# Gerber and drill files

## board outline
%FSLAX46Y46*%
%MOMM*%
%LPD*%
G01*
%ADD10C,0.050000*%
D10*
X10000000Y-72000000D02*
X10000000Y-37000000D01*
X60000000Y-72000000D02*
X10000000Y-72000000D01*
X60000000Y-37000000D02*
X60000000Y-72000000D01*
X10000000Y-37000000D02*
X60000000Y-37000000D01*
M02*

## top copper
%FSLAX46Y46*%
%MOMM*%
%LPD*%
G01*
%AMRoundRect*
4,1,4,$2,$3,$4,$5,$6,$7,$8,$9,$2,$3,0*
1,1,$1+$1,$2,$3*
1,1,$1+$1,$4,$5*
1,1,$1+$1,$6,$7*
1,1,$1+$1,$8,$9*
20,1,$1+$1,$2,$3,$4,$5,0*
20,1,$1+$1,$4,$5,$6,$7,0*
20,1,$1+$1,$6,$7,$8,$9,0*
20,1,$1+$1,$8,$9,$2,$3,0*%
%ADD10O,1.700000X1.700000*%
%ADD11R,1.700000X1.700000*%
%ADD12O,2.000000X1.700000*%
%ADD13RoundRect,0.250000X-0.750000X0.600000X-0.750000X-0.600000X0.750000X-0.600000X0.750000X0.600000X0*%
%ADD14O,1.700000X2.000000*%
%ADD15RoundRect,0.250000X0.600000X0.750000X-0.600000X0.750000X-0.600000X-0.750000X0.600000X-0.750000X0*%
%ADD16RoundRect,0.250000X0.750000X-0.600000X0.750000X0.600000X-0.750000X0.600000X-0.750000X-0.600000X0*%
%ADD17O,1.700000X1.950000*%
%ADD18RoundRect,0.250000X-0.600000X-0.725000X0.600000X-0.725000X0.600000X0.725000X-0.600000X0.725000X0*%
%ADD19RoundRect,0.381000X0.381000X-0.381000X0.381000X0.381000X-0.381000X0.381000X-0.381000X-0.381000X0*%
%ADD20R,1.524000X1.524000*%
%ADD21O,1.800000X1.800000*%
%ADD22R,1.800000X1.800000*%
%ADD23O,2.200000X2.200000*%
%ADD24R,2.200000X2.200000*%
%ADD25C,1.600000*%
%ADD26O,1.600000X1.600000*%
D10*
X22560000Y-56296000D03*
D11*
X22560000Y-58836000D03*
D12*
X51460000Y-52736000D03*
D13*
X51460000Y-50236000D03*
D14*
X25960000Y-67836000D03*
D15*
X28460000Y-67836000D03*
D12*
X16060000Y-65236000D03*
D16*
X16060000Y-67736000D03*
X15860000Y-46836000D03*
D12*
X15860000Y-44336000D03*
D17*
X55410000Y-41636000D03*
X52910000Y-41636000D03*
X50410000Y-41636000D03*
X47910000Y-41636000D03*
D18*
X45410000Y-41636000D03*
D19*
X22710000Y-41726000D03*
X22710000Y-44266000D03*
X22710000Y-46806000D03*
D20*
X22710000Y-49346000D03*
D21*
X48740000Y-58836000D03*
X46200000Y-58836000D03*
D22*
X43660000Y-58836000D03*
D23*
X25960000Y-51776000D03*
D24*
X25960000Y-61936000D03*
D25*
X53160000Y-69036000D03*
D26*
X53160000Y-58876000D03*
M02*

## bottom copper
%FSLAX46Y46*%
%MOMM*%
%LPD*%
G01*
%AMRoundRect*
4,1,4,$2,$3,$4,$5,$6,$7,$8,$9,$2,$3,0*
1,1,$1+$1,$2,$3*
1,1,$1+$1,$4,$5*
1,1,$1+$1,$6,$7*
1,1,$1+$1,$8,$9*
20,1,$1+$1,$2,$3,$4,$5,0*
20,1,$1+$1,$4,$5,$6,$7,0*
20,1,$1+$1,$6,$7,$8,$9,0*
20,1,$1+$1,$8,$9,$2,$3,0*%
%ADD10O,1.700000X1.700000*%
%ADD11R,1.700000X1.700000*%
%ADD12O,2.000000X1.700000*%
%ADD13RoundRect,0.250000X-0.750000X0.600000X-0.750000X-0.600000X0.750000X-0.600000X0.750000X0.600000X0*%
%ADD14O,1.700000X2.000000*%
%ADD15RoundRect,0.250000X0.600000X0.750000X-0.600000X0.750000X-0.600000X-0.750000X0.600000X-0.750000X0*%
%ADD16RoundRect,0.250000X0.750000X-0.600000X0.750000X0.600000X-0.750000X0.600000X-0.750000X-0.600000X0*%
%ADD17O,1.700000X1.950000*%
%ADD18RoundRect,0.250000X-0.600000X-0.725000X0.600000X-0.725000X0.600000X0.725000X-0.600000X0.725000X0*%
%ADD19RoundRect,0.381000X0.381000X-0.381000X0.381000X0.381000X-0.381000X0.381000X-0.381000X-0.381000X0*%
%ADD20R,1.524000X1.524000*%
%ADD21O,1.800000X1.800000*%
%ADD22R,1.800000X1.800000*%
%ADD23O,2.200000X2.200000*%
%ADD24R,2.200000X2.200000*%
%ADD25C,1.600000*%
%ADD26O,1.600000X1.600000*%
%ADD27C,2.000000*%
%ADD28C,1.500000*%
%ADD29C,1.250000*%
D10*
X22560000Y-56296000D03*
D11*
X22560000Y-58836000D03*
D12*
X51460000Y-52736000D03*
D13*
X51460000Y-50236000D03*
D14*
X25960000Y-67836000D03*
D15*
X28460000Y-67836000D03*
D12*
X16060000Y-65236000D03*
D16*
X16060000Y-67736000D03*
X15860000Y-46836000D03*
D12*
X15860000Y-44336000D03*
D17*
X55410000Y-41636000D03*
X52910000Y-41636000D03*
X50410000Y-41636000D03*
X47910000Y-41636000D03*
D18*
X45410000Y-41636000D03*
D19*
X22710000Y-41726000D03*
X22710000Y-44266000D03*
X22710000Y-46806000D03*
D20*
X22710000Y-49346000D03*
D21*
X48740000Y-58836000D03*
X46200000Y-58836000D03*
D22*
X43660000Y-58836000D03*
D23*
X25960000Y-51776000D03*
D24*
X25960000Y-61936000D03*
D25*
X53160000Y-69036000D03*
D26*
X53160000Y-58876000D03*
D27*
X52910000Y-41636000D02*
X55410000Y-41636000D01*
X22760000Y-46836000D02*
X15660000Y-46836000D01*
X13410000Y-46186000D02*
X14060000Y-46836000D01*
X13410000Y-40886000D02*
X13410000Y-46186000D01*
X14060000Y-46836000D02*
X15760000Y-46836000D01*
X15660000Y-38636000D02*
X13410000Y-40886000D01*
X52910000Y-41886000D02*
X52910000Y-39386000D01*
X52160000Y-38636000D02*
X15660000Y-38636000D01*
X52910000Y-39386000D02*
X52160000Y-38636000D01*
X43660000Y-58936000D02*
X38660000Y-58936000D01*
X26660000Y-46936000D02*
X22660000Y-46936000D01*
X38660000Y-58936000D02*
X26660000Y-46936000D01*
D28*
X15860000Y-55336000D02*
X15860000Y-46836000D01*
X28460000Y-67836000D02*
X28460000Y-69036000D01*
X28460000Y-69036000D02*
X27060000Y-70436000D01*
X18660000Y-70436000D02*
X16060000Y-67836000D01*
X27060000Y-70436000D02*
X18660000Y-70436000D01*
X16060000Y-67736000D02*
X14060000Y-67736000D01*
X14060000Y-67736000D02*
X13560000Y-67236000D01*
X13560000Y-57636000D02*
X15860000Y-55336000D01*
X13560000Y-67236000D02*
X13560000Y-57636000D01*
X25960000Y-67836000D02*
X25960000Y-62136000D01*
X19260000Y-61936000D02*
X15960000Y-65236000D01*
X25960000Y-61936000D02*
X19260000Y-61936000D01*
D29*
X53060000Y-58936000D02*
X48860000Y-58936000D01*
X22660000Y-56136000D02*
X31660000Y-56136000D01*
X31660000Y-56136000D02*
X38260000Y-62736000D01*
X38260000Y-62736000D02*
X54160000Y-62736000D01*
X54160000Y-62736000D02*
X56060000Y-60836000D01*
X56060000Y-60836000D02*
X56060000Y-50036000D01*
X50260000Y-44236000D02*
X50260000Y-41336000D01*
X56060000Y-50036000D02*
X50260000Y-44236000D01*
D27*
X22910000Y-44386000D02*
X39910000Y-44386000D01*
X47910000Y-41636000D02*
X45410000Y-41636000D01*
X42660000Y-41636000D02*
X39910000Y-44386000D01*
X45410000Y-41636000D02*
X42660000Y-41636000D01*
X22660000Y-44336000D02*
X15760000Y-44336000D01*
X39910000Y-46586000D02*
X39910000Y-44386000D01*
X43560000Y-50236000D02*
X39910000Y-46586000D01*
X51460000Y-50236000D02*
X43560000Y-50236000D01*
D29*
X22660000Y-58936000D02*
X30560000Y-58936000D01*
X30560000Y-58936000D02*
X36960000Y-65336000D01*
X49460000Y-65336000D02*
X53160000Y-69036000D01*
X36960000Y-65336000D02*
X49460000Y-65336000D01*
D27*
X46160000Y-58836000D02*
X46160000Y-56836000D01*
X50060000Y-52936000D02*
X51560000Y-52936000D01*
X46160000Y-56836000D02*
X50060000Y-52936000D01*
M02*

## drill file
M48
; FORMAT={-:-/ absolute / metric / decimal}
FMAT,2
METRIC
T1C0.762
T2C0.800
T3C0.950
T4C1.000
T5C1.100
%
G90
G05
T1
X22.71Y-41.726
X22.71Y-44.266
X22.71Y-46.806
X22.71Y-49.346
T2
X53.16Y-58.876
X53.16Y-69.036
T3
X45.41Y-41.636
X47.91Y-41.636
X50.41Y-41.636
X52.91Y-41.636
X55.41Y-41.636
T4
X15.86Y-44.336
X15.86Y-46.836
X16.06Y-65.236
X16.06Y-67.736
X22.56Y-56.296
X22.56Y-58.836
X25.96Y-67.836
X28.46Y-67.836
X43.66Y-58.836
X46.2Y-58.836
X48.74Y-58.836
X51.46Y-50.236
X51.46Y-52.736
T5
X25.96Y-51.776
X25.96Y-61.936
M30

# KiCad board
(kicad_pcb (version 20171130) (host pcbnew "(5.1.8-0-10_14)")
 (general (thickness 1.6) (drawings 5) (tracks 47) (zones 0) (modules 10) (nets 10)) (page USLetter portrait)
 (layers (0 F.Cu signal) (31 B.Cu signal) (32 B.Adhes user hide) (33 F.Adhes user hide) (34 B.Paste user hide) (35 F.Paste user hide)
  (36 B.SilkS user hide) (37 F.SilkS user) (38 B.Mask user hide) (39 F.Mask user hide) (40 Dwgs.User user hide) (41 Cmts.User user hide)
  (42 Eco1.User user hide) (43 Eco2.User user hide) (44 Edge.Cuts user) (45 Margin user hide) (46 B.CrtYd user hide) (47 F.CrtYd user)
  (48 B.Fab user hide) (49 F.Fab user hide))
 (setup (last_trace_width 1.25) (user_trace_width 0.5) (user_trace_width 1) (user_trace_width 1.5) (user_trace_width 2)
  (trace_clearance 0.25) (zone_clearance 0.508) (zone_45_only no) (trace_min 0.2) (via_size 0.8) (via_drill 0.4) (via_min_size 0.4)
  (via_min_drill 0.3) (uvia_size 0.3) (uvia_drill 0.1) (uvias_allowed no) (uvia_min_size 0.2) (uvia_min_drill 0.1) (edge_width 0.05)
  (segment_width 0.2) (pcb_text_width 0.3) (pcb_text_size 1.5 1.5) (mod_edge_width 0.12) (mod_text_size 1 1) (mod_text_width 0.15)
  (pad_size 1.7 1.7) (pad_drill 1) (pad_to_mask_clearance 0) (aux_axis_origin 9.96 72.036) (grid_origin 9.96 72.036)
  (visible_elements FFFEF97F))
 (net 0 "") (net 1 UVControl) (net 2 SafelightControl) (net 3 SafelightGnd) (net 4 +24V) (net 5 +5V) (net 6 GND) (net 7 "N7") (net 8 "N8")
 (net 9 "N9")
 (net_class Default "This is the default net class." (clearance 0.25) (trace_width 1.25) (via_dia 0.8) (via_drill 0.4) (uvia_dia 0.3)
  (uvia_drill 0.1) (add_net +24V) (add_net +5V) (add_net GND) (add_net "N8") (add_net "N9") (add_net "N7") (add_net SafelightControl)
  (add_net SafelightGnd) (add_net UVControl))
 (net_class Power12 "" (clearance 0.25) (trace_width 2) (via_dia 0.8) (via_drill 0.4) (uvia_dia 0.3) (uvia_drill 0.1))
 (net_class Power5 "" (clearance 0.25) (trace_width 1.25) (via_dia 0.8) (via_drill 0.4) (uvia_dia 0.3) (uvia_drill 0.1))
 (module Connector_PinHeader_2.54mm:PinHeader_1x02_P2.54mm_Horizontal (layer F.Cu) (at 22.56 58.836 180)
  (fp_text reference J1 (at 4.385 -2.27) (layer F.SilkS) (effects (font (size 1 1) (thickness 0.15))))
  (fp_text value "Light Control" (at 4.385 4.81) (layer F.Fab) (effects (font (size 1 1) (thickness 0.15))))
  (pad 2 thru_hole oval (at 0 2.54 180) (size 1.7 1.7) (drill 1) (layers *.Cu *.Mask) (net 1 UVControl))
  (pad 1 thru_hole rect (at 0 0 180) (size 1.7 1.7) (drill 1) (layers *.Cu *.Mask) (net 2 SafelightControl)))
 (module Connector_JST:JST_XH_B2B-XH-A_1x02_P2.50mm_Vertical (layer F.Cu) (at 51.46 50.236 270)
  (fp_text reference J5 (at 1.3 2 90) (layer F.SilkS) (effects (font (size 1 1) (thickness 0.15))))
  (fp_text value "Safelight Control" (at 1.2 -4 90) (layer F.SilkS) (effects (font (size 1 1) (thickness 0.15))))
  (pad 2 thru_hole oval (at 2.5 0 270) (size 1.7 2) (drill 1) (layers *.Cu *.Mask) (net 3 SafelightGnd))
  (pad 1 thru_hole roundrect (at 0 0 270) (size 1.7 2) (drill 1) (layers *.Cu *.Mask) (roundrect_rratio 0.1470588235294118) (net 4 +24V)))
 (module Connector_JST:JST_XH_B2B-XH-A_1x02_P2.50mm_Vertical (layer F.Cu) (at 28.46 67.836 180)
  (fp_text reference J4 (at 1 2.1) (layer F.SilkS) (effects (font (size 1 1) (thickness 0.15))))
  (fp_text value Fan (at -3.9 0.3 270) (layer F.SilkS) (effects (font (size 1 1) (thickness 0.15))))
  (pad 2 thru_hole oval (at 2.5 0 180) (size 1.7 2) (drill 1) (layers *.Cu *.Mask) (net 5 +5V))
  (pad 1 thru_hole roundrect (at 0 0 180) (size 1.7 2) (drill 1) (layers *.Cu *.Mask) (roundrect_rratio 0.1470588235294118) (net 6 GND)))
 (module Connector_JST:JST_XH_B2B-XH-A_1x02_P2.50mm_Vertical (layer F.Cu) (at 16.06 67.736 90)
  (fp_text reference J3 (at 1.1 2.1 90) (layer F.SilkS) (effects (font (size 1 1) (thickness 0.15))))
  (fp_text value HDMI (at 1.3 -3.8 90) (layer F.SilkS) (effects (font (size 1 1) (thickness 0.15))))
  (pad 2 thru_hole oval (at 2.5 0 90) (size 1.7 2) (drill 1) (layers *.Cu *.Mask) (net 5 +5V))
  (pad 1 thru_hole roundrect (at 0 0 90) (size 1.7 2) (drill 1) (layers *.Cu *.Mask) (roundrect_rratio 0.1470588235294118) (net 6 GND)))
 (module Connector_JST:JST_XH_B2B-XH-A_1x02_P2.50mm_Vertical (layer F.Cu) (at 15.86 46.836 90)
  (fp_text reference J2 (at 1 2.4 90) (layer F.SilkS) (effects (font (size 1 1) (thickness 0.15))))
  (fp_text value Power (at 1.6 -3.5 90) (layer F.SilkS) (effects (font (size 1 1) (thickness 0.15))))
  (pad 1 thru_hole roundrect (at 0 0 90) (size 1.7 2) (drill 1) (layers *.Cu *.Mask) (roundrect_rratio 0.1470588235294118) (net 6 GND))
  (pad 2 thru_hole oval (at 2.5 0 90) (size 1.7 2) (drill 1) (layers *.Cu *.Mask) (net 4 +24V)))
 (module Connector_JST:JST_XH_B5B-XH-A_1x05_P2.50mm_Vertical (layer F.Cu) (at 45.41 41.636)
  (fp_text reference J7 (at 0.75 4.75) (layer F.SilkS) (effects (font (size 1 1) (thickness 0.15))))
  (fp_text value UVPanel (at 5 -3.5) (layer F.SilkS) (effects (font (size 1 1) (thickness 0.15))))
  (pad 5 thru_hole oval (at 10 0) (size 1.7 1.95) (drill 0.95) (layers *.Cu *.Mask) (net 6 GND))
  (pad 4 thru_hole oval (at 7.5 0) (size 1.7 1.95) (drill 0.95) (layers *.Cu *.Mask) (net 6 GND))
  (pad 3 thru_hole oval (at 5 0) (size 1.7 1.95) (drill 0.95) (layers *.Cu *.Mask) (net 1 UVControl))
  (pad 2 thru_hole oval (at 2.5 0) (size 1.7 1.95) (drill 0.95) (layers *.Cu *.Mask) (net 4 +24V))
  (pad 1 thru_hole roundrect (at 0 0) (size 1.7 1.95) (drill 0.95) (layers *.Cu *.Mask) (roundrect_rratio 0.1470588235294118) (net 4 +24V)))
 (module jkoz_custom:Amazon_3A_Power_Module (layer F.Cu) (at 30.66 45.636 90)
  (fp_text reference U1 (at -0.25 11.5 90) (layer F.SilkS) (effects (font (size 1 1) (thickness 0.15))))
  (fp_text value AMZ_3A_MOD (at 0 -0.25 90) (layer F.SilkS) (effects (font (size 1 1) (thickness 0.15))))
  (pad 4 thru_hole roundrect (at 3.91 -7.95 90) (size 1.524 1.524) (drill 0.762) (layers *.Cu *.Mask) (roundrect_rratio 0.25) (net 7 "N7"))
  (pad 3 thru_hole roundrect (at 1.37 -7.95 90) (size 1.524 1.524) (drill 0.762) (layers *.Cu *.Mask) (roundrect_rratio 0.25) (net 4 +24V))
  (pad 2 thru_hole roundrect (at -1.17 -7.95 90) (size 1.524 1.524) (drill 0.762) (layers *.Cu *.Mask) (roundrect_rratio 0.25) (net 6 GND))
  (pad 1 thru_hole rect (at -3.71 -7.95 90) (size 1.524 1.524) (drill 0.762) (layers *.Cu *.Mask) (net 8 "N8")))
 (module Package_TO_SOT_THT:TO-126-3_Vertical (layer F.Cu) (at 43.66 58.836)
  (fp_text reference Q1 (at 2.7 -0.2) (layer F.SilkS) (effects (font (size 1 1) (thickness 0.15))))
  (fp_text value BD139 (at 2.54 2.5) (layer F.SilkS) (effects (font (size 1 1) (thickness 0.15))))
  (pad 3 thru_hole oval (at 5.08 0) (size 1.8 1.8) (drill 1) (layers *.Cu *.Mask) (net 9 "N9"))
  (pad 2 thru_hole oval (at 2.54 0) (size 1.8 1.8) (drill 1) (layers *.Cu *.Mask) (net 3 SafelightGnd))
  (pad 1 thru_hole rect (at 0 0) (size 1.8 1.8) (drill 1) (layers *.Cu *.Mask) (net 6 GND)))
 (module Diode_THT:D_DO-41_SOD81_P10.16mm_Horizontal (layer F.Cu) (at 25.96 61.936 90)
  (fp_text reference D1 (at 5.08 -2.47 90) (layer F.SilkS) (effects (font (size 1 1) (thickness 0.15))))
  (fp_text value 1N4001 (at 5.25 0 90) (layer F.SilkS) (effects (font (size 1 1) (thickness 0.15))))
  (pad 2 thru_hole oval (at 10.16 0 90) (size 2.2 2.2) (drill 1.1) (layers *.Cu *.Mask) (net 8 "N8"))
  (pad 1 thru_hole rect (at 0 0 90) (size 2.2 2.2) (drill 1.1) (layers *.Cu *.Mask) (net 5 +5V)))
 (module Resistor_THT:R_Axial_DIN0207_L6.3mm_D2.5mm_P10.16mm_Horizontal (layer F.Cu) (at 53.16 69.036 90)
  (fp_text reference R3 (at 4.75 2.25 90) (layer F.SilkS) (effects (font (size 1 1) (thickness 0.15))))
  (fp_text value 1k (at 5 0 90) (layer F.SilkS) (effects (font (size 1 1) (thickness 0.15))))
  (pad 1 thru_hole circle (at 0 0 90) (size 1.6 1.6) (drill 0.8) (layers *.Cu *.Mask) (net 2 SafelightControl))
  (pad 2 thru_hole oval (at 10.16 0 90) (size 1.6 1.6) (drill 0.8) (layers *.Cu *.Mask) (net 9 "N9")))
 (gr_line (start 10 72) (end 10 37) (layer Edge.Cuts) (width 0.05))
 (gr_line (start 60 72) (end 10 72) (layer Edge.Cuts) (width 0.05))
 (gr_line (start 60 37) (end 60 72) (layer Edge.Cuts) (width 0.05))
 (gr_line (start 10 37) (end 60 37) (layer Edge.Cuts) (width 0.05))
 (segment (start 52.91 41.636) (end 55.41 41.636) (width 2) (layer B.Cu) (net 6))
 (segment (start 22.76 46.836) (end 15.66 46.836) (width 2) (layer B.Cu) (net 6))
 (segment (start 13.41 46.186) (end 14.06 46.836) (width 2) (layer B.Cu) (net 6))
 (segment (start 13.41 40.886) (end 13.41 46.186) (width 2) (layer B.Cu) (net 6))
 (segment (start 14.06 46.836) (end 15.76 46.836) (width 2) (layer B.Cu) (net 6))
 (segment (start 15.66 38.636) (end 13.41 40.886) (width 2) (layer B.Cu) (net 6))
 (segment (start 52.91 41.886) (end 52.91 39.386) (width 2) (layer B.Cu) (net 6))
 (segment (start 52.16 38.636) (end 15.66 38.636) (width 2) (layer B.Cu) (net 6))
 (segment (start 52.91 39.386) (end 52.16 38.636) (width 2) (layer B.Cu) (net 6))
 (segment (start 43.66 58.936) (end 38.66 58.936) (width 2) (layer B.Cu) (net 6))
 (segment (start 26.66 46.936) (end 22.66 46.936) (width 2) (layer B.Cu) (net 6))
 (segment (start 38.66 58.936) (end 26.66 46.936) (width 2) (layer B.Cu) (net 6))
 (segment (start 15.86 55.336) (end 15.86 46.836) (width 1.5) (layer B.Cu) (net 6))
 (segment (start 28.46 67.836) (end 28.46 69.036) (width 1.5) (layer B.Cu) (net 6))
 (segment (start 28.46 69.036) (end 27.06 70.436) (width 1.5) (layer B.Cu) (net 6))
 (segment (start 18.66 70.436) (end 16.06 67.836) (width 1.5) (layer B.Cu) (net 6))
 (segment (start 27.06 70.436) (end 18.66 70.436) (width 1.5) (layer B.Cu) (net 6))
 (segment (start 16.06 67.736) (end 14.06 67.736) (width 1.5) (layer B.Cu) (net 6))
 (segment (start 14.06 67.736) (end 13.56 67.236) (width 1.5) (layer B.Cu) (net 6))
 (segment (start 13.56 57.636) (end 15.86 55.336) (width 1.5) (layer B.Cu) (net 6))
 (segment (start 13.56 67.236) (end 13.56 57.636) (width 1.5) (layer B.Cu) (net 6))
 (segment (start 25.96 67.836) (end 25.96 62.136) (width 1.5) (layer B.Cu) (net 5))
 (segment (start 19.26 61.936) (end 15.96 65.236) (width 1.5) (layer B.Cu) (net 5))
 (segment (start 25.96 61.936) (end 19.26 61.936) (width 1.5) (layer B.Cu) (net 5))
 (segment (start 53.06 58.936) (end 48.86 58.936) (width 1.25) (layer B.Cu) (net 9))
 (segment (start 22.66 56.136) (end 31.66 56.136) (width 1.25) (layer B.Cu) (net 1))
 (segment (start 31.66 56.136) (end 38.26 62.736) (width 1.25) (layer B.Cu) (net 1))
 (segment (start 38.26 62.736) (end 54.16 62.736) (width 1.25) (layer B.Cu) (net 1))
 (segment (start 54.16 62.736) (end 56.06 60.836) (width 1.25) (layer B.Cu) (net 1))
 (segment (start 56.06 60.836) (end 56.06 50.036) (width 1.25) (layer B.Cu) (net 1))
 (segment (start 50.26 44.236) (end 50.26 41.336) (width 1.25) (layer B.Cu) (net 1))
 (segment (start 56.06 50.036) (end 50.26 44.236) (width 1.25) (layer B.Cu) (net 1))
 (segment (start 22.91 44.386) (end 39.91 44.386) (width 2) (layer B.Cu) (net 4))
 (segment (start 47.91 41.636) (end 45.41 41.636) (width 2) (layer B.Cu) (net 4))
 (segment (start 42.66 41.636) (end 39.91 44.386) (width 2) (layer B.Cu) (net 4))
 (segment (start 45.41 41.636) (end 42.66 41.636) (width 2) (layer B.Cu) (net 4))
 (segment (start 22.66 44.336) (end 15.76 44.336) (width 2) (layer B.Cu) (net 4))
 (segment (start 39.91 46.586) (end 39.91 44.386) (width 2) (layer B.Cu) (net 4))
 (segment (start 43.56 50.236) (end 39.91 46.586) (width 2) (layer B.Cu) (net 4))
 (segment (start 51.46 50.236) (end 43.56 50.236) (width 2) (layer B.Cu) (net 4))
 (segment (start 22.66 58.936) (end 30.56 58.936) (width 1.25) (layer B.Cu) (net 2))
 (segment (start 30.56 58.936) (end 36.96 65.336) (width 1.25) (layer B.Cu) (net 2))
 (segment (start 49.46 65.336) (end 53.16 69.036) (width 1.25) (layer B.Cu) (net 2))
 (segment (start 36.96 65.336) (end 49.46 65.336) (width 1.25) (layer B.Cu) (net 2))
 (segment (start 46.16 58.836) (end 46.16 56.836) (width 2) (layer B.Cu) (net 3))
 (segment (start 50.06 52.936) (end 51.56 52.936) (width 2) (layer B.Cu) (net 3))
 (segment (start 46.16 56.836) (end 50.06 52.936) (width 2) (layer B.Cu) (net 3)))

